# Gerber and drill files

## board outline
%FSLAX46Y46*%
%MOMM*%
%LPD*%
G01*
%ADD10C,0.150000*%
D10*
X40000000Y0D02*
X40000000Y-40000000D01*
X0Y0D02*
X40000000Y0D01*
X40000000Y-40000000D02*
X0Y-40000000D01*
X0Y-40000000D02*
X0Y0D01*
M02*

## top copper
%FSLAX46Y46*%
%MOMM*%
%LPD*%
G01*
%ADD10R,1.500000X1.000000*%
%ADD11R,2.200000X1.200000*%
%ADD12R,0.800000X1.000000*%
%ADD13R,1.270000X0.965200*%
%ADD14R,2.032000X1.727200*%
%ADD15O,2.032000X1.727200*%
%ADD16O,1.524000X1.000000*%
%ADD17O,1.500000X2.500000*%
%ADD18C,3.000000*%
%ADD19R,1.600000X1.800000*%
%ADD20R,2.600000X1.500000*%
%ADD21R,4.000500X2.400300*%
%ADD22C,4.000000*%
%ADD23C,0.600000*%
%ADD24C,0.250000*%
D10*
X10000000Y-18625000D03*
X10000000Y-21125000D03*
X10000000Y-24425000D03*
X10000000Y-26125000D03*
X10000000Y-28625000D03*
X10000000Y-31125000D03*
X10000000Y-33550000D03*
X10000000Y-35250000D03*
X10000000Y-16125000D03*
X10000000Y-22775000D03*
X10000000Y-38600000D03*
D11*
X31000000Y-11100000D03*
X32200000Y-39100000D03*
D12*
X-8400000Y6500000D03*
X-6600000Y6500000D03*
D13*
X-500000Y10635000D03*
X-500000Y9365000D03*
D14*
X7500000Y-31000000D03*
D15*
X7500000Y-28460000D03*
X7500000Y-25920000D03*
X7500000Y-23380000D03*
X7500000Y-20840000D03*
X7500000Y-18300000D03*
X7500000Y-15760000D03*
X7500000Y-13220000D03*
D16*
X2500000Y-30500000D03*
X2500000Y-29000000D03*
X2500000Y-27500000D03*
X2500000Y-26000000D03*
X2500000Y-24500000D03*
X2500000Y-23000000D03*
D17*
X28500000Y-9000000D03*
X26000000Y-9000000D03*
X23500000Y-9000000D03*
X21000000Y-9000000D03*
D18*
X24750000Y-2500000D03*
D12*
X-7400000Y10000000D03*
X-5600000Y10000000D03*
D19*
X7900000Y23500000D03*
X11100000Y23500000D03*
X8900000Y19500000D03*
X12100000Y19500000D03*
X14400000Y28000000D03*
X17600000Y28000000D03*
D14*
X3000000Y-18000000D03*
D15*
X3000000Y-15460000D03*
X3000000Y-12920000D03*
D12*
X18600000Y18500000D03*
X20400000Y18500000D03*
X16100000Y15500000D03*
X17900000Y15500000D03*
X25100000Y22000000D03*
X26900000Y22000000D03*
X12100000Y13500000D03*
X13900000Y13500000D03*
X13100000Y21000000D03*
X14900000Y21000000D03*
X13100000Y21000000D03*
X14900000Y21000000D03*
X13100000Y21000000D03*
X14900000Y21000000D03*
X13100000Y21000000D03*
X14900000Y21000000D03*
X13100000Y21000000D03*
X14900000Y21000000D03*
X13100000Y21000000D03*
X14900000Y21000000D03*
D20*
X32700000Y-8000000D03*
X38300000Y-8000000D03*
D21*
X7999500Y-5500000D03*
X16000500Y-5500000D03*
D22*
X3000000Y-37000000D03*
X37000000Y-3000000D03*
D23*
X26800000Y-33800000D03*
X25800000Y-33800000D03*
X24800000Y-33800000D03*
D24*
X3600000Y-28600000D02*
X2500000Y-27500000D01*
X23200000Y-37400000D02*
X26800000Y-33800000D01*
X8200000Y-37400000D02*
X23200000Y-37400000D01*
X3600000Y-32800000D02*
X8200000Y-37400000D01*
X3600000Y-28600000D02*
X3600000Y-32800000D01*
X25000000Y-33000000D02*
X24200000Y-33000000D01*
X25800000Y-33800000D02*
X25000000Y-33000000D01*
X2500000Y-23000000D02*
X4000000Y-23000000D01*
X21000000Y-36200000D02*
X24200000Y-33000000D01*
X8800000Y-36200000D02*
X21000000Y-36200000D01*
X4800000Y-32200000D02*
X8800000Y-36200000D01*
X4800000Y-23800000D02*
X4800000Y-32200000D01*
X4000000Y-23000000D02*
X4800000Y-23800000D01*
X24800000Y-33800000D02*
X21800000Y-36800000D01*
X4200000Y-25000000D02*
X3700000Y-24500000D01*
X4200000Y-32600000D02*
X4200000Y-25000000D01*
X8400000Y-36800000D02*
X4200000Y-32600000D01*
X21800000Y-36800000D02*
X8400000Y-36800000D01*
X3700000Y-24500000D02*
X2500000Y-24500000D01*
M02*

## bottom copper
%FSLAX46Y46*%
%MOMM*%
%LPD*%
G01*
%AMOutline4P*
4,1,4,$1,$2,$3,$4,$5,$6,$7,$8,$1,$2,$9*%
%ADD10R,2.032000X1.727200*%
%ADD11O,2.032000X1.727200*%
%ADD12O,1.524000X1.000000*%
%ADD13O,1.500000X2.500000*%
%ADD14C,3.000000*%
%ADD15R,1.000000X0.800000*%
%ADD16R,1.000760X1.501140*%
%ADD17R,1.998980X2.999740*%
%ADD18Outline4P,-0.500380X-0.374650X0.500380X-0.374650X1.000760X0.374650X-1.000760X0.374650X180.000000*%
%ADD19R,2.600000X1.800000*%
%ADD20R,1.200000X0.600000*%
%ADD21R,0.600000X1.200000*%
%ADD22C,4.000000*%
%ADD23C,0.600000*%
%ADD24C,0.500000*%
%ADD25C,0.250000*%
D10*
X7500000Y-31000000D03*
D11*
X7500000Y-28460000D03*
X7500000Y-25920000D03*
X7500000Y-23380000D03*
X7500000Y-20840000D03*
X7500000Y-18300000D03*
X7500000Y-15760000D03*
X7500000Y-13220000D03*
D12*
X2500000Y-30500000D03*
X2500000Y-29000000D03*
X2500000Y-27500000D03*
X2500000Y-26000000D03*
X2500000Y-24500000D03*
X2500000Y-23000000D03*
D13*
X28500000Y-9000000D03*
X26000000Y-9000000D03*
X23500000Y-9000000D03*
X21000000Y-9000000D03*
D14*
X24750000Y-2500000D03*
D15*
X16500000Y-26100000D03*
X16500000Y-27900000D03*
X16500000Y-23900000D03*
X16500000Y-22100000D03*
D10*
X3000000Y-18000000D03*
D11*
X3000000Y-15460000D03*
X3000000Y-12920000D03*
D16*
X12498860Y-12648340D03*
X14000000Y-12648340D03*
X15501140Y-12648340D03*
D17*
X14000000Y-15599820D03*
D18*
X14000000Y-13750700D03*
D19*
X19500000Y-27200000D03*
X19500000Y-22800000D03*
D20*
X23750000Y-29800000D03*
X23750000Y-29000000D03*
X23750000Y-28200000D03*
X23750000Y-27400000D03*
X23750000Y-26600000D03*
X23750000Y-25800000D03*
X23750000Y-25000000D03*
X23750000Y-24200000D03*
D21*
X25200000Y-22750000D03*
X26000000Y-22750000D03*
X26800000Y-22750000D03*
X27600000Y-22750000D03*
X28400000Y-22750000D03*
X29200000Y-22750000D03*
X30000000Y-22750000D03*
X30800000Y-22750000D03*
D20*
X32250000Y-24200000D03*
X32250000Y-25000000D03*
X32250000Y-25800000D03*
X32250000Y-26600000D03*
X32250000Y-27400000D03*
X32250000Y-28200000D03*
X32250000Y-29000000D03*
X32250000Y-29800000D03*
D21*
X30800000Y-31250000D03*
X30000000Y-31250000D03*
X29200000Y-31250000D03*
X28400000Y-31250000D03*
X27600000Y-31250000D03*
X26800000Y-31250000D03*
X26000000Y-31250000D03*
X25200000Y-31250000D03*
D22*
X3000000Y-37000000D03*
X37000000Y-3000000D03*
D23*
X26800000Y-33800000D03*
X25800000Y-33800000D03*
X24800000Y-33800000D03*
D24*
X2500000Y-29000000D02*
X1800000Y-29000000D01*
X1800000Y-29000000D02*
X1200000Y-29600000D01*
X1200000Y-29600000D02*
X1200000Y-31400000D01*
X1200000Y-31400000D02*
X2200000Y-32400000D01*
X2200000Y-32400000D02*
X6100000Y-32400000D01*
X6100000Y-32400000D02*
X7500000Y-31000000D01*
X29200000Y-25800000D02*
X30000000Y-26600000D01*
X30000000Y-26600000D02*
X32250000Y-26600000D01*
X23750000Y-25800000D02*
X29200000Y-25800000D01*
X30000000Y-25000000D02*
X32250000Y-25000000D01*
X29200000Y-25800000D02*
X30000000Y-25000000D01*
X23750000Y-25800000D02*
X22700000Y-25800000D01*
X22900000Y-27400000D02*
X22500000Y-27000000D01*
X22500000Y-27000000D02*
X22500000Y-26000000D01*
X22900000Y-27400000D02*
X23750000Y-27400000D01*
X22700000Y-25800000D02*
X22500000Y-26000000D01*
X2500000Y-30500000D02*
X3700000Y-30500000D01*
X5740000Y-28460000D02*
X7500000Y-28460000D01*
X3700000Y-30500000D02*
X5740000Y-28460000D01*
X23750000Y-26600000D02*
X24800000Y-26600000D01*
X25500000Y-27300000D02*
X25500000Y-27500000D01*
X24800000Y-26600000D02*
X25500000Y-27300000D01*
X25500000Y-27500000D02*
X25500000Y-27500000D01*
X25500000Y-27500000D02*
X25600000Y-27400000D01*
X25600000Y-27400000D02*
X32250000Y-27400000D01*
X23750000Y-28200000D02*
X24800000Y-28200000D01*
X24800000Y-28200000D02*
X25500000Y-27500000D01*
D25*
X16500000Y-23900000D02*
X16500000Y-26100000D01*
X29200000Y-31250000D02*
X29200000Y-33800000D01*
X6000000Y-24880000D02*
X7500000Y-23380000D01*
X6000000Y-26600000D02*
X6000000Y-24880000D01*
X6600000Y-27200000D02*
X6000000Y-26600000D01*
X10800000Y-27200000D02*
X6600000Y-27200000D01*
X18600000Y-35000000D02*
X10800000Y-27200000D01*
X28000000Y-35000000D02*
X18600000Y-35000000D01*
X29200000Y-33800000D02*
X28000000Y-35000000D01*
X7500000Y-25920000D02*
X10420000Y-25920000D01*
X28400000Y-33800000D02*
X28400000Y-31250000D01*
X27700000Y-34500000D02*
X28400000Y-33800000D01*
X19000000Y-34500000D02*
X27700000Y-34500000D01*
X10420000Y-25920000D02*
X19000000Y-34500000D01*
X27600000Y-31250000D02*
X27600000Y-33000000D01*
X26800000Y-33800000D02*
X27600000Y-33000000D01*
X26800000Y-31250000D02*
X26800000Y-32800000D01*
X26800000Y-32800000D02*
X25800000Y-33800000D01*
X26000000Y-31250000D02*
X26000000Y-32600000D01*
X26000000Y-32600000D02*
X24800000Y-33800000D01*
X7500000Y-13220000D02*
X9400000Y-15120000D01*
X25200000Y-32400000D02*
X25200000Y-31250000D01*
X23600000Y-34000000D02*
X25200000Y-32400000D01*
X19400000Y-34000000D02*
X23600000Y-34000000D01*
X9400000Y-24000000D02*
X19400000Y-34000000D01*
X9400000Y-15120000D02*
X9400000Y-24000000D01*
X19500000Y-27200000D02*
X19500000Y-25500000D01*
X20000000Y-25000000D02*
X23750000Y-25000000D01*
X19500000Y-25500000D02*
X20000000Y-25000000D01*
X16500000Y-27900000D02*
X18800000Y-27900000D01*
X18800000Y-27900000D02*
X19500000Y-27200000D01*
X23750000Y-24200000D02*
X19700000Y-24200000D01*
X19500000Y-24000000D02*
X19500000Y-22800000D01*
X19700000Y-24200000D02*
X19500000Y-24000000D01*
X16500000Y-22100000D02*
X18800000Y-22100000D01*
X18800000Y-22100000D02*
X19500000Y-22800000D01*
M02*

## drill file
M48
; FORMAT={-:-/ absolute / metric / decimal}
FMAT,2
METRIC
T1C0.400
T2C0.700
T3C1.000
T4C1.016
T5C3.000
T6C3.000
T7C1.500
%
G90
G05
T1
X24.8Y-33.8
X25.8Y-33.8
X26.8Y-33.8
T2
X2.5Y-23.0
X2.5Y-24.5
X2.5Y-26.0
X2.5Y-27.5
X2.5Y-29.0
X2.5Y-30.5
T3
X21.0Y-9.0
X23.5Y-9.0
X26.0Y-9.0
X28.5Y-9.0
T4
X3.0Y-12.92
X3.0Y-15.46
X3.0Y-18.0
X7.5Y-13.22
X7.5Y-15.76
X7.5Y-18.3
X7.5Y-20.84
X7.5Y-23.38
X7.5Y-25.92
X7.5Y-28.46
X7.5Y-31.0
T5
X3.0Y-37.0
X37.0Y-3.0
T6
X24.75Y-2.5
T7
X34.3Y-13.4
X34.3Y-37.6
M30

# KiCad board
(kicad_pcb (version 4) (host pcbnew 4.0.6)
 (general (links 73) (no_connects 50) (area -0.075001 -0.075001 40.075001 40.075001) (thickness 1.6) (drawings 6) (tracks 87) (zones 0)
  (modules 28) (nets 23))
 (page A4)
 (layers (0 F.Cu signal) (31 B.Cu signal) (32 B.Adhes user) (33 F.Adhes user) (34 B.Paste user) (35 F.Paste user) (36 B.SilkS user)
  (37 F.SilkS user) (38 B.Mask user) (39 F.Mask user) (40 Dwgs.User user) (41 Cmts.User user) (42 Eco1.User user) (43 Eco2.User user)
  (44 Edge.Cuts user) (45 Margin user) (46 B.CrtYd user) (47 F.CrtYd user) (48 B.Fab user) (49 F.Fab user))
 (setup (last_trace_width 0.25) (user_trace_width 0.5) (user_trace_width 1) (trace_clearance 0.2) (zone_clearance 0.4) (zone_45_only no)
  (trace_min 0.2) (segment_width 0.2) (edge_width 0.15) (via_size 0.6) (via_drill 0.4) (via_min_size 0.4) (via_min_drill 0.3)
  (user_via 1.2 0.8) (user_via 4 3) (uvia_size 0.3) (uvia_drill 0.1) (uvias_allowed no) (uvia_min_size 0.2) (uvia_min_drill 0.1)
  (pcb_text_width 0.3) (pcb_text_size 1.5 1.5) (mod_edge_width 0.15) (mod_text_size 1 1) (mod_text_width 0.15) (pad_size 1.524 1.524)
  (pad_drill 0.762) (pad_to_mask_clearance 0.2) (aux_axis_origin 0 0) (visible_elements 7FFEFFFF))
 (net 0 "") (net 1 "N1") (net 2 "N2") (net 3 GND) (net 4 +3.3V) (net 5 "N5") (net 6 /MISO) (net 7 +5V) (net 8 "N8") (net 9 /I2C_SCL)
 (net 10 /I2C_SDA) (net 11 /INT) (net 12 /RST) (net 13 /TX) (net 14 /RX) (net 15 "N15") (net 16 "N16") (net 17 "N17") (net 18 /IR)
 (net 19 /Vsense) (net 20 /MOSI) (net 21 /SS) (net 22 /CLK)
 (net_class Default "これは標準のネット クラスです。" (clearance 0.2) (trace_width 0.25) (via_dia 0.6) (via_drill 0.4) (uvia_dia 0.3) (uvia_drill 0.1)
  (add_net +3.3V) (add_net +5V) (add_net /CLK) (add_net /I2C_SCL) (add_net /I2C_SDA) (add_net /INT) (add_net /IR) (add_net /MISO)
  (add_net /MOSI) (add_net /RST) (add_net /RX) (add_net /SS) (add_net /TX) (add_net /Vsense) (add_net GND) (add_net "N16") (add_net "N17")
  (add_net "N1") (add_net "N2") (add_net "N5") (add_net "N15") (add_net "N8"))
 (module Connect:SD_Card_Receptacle (layer F.Cu) (at 10 25.5 90)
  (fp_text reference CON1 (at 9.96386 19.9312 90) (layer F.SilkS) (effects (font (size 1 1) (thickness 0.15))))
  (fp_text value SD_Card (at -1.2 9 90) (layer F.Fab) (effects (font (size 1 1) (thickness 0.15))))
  (pad 1 smd rect (at 6.875 0 90) (size 1 1.5) (layers F.Cu F.Paste F.Mask) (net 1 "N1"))
  (pad 2 smd rect (at 4.375 0 90) (size 1 1.5) (layers F.Cu F.Paste F.Mask) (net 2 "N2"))
  (pad 3 smd rect (at 1.075 0 90) (size 1 1.5) (layers F.Cu F.Paste F.Mask) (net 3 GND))
  (pad 4 smd rect (at -0.625 0 90) (size 1 1.5) (layers F.Cu F.Paste F.Mask) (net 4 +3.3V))
  (pad 5 smd rect (at -3.125 0 90) (size 1 1.5) (layers F.Cu F.Paste F.Mask) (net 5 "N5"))
  (pad 6 smd rect (at -5.625 0 90) (size 1 1.5) (layers F.Cu F.Paste F.Mask) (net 3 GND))
  (pad 7 smd rect (at -8.05 0 90) (size 1 1.5) (layers F.Cu F.Paste F.Mask) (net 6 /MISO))
  (pad 8 smd rect (at -9.75 0 90) (size 1 1.5) (layers F.Cu F.Paste F.Mask))
  (pad 9 smd rect (at 9.375 0 90) (size 1 1.5) (layers F.Cu F.Paste F.Mask))
  (pad 10 smd rect (at 2.725 0 90) (size 1 1.5) (layers F.Cu F.Paste F.Mask))
  (pad 11 smd rect (at -13.1 0 90) (size 1 1.5) (layers F.Cu F.Paste F.Mask))
  (pad 12 smd rect (at 14.4 21 90) (size 1.2 2.2) (layers F.Cu F.Paste F.Mask) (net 3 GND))
  (pad 13 smd rect (at -13.6 22.2 90) (size 1.2 2.2) (layers F.Cu F.Paste F.Mask) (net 3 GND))
  (pad "" np_thru_hole circle (at 12.1 24.3 90) (size 1.5 1.5) (drill 1.5) (layers *.Cu *.Mask F.SilkS))
  (pad "" np_thru_hole circle (at -12.1 24.3 90) (size 1.5 1.5) (drill 1.5) (layers *.Cu *.Mask F.SilkS)))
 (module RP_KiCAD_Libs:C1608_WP (layer F.Cu) (at -7.5 -6.5)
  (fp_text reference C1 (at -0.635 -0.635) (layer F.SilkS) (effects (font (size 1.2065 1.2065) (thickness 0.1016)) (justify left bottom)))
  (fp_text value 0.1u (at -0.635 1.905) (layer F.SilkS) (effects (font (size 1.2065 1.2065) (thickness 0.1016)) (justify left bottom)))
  (pad 1 smd rect (at -0.9 0) (size 0.8 1) (layers F.Cu F.Paste F.Mask) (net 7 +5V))
  (pad 2 smd rect (at 0.9 0) (size 0.8 1) (layers F.Cu F.Paste F.Mask) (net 3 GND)))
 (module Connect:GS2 (layer F.Cu) (at -0.5 -10)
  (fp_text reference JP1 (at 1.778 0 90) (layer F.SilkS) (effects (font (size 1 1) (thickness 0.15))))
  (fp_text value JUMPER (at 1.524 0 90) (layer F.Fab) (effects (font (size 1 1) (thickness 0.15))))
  (pad 1 smd rect (at 0 -0.635) (size 1.27 0.9652) (layers F.Cu F.Paste F.Mask) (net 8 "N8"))
  (pad 2 smd rect (at 0 0.635) (size 1.27 0.9652) (layers F.Cu F.Paste F.Mask) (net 3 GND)))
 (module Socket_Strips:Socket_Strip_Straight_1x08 (layer F.Cu) (at 7.5 31 90)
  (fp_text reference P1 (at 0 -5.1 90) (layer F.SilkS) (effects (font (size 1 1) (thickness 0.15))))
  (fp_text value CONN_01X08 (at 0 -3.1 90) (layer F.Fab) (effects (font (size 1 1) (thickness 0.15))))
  (pad 1 thru_hole rect (at 0 0 90) (size 1.7272 2.032) (drill 1.016) (layers *.Cu *.Mask F.SilkS) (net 7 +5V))
  (pad 2 thru_hole oval (at 2.54 0 90) (size 1.7272 2.032) (drill 1.016) (layers *.Cu *.Mask F.SilkS) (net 3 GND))
  (pad 3 thru_hole oval (at 5.08 0 90) (size 1.7272 2.032) (drill 1.016) (layers *.Cu *.Mask F.SilkS) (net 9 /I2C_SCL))
  (pad 4 thru_hole oval (at 7.62 0 90) (size 1.7272 2.032) (drill 1.016) (layers *.Cu *.Mask F.SilkS) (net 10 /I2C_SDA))
  (pad 5 thru_hole oval (at 10.16 0 90) (size 1.7272 2.032) (drill 1.016) (layers *.Cu *.Mask F.SilkS))
  (pad 6 thru_hole oval (at 12.7 0 90) (size 1.7272 2.032) (drill 1.016) (layers *.Cu *.Mask F.SilkS))
  (pad 7 thru_hole oval (at 15.24 0 90) (size 1.7272 2.032) (drill 1.016) (layers *.Cu *.Mask F.SilkS) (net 8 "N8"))
  (pad 8 thru_hole oval (at 17.78 0 90) (size 1.7272 2.032) (drill 1.016) (layers *.Cu *.Mask F.SilkS) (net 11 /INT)))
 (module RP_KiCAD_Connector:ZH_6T (layer F.Cu) (at 2.5 30.5 90)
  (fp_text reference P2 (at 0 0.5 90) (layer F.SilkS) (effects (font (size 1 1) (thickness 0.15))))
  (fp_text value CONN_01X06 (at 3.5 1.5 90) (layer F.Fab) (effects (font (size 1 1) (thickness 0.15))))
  (pad 1 thru_hole oval (at 0 0 90) (size 1 1.524) (drill 0.7) (layers *.Cu *.Mask) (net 3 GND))
  (pad 2 thru_hole oval (at 1.5 0 90) (size 1 1.524) (drill 0.7) (layers *.Cu *.Mask) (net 7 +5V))
  (pad 3 thru_hole oval (at 3 0 90) (size 1 1.524) (drill 0.7) (layers *.Cu *.Mask) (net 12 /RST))
  (pad 4 thru_hole oval (at 4.5 0 90) (size 1 1.524) (drill 0.7) (layers *.Cu *.Mask))
  (pad 5 thru_hole oval (at 6 0 90) (size 1 1.524) (drill 0.7) (layers *.Cu *.Mask) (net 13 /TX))
  (pad 6 thru_hole oval (at 7.5 0 90) (size 1 1.524) (drill 0.7) (layers *.Cu *.Mask) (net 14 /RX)))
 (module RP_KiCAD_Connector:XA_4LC (layer F.Cu) (at 28.5 9 180)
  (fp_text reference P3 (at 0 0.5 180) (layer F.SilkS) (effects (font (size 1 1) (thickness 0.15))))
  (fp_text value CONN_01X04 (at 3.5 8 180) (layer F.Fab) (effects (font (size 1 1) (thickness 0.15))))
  (pad 1 thru_hole oval (at 0 0 180) (size 1.5 2.5) (drill 1) (layers *.Cu *.Mask F.SilkS) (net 3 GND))
  (pad 2 thru_hole oval (at 2.5 0 180) (size 1.5 2.5) (drill 1) (layers *.Cu *.Mask F.SilkS) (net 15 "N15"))
  (pad 3 thru_hole oval (at 5 0 180) (size 1.5 2.5) (drill 1) (layers *.Cu *.Mask F.SilkS) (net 14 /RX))
  (pad 4 thru_hole oval (at 7.5 0 180) (size 1.5 2.5) (drill 1) (layers *.Cu *.Mask F.SilkS) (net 13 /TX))
  (pad "" thru_hole circle (at 3.75 6.5 180) (size 3 3) (drill 3) (layers *.Cu *.Mask F.SilkS) (clearance -0.3)))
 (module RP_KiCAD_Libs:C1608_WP (layer F.Cu) (at -6.5 -10)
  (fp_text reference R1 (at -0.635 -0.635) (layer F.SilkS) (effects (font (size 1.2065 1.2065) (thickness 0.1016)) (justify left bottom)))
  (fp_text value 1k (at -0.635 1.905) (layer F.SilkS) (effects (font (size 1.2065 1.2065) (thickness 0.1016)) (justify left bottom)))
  (pad 1 smd rect (at -0.9 0) (size 0.8 1) (layers F.Cu F.Paste F.Mask) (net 7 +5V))
  (pad 2 smd rect (at 0.9 0) (size 0.8 1) (layers F.Cu F.Paste F.Mask) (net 12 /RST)))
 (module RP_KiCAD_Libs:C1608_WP (layer B.Cu) (at 16.5 27 270)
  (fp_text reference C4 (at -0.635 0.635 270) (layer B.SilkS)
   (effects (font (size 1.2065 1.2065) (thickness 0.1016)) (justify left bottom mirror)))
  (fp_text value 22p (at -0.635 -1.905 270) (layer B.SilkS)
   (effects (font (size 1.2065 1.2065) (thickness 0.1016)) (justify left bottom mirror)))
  (pad 1 smd rect (at -0.9 0 270) (size 0.8 1) (layers B.Cu B.Paste B.Mask) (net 3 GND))
  (pad 2 smd rect (at 0.9 0 270) (size 0.8 1) (layers B.Cu B.Paste B.Mask) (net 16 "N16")))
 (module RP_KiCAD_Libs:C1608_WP (layer B.Cu) (at 16.5 23 90)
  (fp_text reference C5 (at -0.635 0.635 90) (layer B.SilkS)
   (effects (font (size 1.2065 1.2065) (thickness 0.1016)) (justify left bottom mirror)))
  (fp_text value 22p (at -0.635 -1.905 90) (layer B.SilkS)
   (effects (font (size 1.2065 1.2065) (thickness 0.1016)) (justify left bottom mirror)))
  (pad 1 smd rect (at -0.9 0 90) (size 0.8 1) (layers B.Cu B.Paste B.Mask) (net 3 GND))
  (pad 2 smd rect (at 0.9 0 90) (size 0.8 1) (layers B.Cu B.Paste B.Mask) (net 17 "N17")))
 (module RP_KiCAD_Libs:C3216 (layer F.Cu) (at 9.5 -23.5)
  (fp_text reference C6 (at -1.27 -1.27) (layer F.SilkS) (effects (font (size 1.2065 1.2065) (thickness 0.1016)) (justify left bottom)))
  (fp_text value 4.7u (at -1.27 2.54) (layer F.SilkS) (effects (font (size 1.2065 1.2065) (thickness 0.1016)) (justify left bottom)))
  (pad 1 smd rect (at -1.6 0) (size 1.6 1.8) (layers F.Cu F.Paste F.Mask) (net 7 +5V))
  (pad 2 smd rect (at 1.6 0) (size 1.6 1.8) (layers F.Cu F.Paste F.Mask) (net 3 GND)))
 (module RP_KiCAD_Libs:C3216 (layer F.Cu) (at 10.5 -19.5)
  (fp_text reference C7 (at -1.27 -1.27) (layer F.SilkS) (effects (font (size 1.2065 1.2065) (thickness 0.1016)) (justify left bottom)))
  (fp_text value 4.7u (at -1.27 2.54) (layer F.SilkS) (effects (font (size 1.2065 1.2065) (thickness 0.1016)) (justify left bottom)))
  (pad 1 smd rect (at -1.6 0) (size 1.6 1.8) (layers F.Cu F.Paste F.Mask) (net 4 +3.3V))
  (pad 2 smd rect (at 1.6 0) (size 1.6 1.8) (layers F.Cu F.Paste F.Mask) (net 3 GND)))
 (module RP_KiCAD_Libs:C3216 (layer F.Cu) (at 16 -28)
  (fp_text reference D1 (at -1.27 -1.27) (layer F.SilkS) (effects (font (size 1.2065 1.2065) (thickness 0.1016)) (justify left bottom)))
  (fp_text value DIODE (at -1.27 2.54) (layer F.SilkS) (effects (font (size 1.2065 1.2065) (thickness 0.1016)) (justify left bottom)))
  (pad 1 smd rect (at -1.6 0) (size 1.6 1.8) (layers F.Cu F.Paste F.Mask) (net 7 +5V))
  (pad 2 smd rect (at 1.6 0) (size 1.6 1.8) (layers F.Cu F.Paste F.Mask) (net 15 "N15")))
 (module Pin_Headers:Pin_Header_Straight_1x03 (layer F.Cu) (at 3 18 180)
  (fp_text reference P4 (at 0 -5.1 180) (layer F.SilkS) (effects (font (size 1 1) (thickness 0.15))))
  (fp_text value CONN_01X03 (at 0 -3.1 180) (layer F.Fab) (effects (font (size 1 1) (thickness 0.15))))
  (pad 1 thru_hole rect (at 0 0 180) (size 2.032 1.7272) (drill 1.016) (layers *.Cu *.Mask F.SilkS) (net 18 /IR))
  (pad 2 thru_hole oval (at 0 2.54 180) (size 2.032 1.7272) (drill 1.016) (layers *.Cu *.Mask F.SilkS) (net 3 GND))
  (pad 3 thru_hole oval (at 0 5.08 180) (size 2.032 1.7272) (drill 1.016) (layers *.Cu *.Mask F.SilkS) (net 7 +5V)))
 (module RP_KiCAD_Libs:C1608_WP (layer F.Cu) (at 19.5 -18.5)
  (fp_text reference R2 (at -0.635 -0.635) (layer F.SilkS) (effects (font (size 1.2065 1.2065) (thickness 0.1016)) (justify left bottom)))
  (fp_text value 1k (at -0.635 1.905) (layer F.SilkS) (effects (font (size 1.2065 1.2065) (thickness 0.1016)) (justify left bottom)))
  (pad 1 smd rect (at -0.9 0) (size 0.8 1) (layers F.Cu F.Paste F.Mask) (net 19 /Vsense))
  (pad 2 smd rect (at 0.9 0) (size 0.8 1) (layers F.Cu F.Paste F.Mask) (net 15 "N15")))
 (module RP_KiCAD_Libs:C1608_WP (layer F.Cu) (at 17 -15.5)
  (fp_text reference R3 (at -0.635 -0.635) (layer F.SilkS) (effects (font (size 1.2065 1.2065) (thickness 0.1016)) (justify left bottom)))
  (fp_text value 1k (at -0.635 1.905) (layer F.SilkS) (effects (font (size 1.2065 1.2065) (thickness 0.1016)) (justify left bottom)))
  (pad 1 smd rect (at -0.9 0) (size 0.8 1) (layers F.Cu F.Paste F.Mask) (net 10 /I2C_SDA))
  (pad 2 smd rect (at 0.9 0) (size 0.8 1) (layers F.Cu F.Paste F.Mask) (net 7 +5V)))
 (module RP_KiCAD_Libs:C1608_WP (layer F.Cu) (at 26 -22)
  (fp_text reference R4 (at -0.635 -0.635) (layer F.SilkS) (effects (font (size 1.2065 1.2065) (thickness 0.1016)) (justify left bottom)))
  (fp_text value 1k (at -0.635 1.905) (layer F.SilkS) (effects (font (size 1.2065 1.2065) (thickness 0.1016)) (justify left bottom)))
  (pad 1 smd rect (at -0.9 0) (size 0.8 1) (layers F.Cu F.Paste F.Mask) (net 9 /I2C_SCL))
  (pad 2 smd rect (at 0.9 0) (size 0.8 1) (layers F.Cu F.Paste F.Mask) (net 7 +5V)))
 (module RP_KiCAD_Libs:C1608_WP (layer F.Cu) (at 13 -13.5)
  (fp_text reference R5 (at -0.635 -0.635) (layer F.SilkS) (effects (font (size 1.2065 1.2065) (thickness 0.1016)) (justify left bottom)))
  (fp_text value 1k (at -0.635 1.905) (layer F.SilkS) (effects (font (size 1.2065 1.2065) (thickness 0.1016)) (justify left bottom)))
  (pad 1 smd rect (at -0.9 0) (size 0.8 1) (layers F.Cu F.Paste F.Mask) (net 3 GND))
  (pad 2 smd rect (at 0.9 0) (size 0.8 1) (layers F.Cu F.Paste F.Mask) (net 19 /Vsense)))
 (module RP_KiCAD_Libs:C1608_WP (layer F.Cu) (at 14 -21)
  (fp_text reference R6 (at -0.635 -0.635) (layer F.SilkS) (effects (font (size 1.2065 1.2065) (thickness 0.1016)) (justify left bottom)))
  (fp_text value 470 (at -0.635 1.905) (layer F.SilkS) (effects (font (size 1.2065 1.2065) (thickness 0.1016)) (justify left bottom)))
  (pad 1 smd rect (at -0.9 0) (size 0.8 1) (layers F.Cu F.Paste F.Mask) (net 2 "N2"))
  (pad 2 smd rect (at 0.9 0) (size 0.8 1) (layers F.Cu F.Paste F.Mask) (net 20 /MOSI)))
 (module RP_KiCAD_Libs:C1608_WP (layer F.Cu) (at 14 -21)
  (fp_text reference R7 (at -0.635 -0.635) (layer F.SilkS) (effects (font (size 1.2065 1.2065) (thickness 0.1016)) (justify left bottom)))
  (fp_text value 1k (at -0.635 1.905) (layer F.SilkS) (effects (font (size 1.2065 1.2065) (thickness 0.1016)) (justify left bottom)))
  (pad 1 smd rect (at -0.9 0) (size 0.8 1) (layers F.Cu F.Paste F.Mask) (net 2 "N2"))
  (pad 2 smd rect (at 0.9 0) (size 0.8 1) (layers F.Cu F.Paste F.Mask) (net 3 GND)))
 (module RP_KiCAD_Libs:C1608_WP (layer F.Cu) (at 14 -21)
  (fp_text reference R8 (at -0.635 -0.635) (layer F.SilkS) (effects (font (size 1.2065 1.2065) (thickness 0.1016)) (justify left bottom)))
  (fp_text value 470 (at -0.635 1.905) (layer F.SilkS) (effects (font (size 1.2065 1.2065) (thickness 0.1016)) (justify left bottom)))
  (pad 1 smd rect (at -0.9 0) (size 0.8 1) (layers F.Cu F.Paste F.Mask) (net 1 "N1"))
  (pad 2 smd rect (at 0.9 0) (size 0.8 1) (layers F.Cu F.Paste F.Mask) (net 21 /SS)))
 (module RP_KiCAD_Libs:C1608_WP (layer F.Cu) (at 14 -21)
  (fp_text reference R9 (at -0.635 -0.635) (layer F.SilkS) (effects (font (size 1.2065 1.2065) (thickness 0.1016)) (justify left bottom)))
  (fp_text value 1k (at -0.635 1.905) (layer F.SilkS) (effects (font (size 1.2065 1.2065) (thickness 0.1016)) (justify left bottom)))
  (pad 1 smd rect (at -0.9 0) (size 0.8 1) (layers F.Cu F.Paste F.Mask) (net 1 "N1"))
  (pad 2 smd rect (at 0.9 0) (size 0.8 1) (layers F.Cu F.Paste F.Mask) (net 3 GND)))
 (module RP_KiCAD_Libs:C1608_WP (layer F.Cu) (at 14 -21)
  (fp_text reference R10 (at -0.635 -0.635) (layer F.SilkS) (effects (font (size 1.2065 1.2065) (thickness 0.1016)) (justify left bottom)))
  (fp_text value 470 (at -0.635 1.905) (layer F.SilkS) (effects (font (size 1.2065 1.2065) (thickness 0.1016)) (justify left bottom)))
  (pad 1 smd rect (at -0.9 0) (size 0.8 1) (layers F.Cu F.Paste F.Mask) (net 5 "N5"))
  (pad 2 smd rect (at 0.9 0) (size 0.8 1) (layers F.Cu F.Paste F.Mask) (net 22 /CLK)))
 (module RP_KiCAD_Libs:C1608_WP (layer F.Cu) (at 14 -21)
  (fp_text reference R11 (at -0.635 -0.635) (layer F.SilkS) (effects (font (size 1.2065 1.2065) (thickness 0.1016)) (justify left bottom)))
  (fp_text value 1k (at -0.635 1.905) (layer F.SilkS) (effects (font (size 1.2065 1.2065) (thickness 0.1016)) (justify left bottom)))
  (pad 1 smd rect (at -0.9 0) (size 0.8 1) (layers F.Cu F.Paste F.Mask) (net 5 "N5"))
  (pad 2 smd rect (at 0.9 0) (size 0.8 1) (layers F.Cu F.Paste F.Mask) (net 3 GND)))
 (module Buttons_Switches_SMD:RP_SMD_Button (layer F.Cu) (at 35.5 8 180)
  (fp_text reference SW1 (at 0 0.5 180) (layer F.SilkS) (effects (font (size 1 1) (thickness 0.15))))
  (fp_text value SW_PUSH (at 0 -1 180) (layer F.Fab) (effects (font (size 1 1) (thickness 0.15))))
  (pad 1 smd rect (at 2.8 0 180) (size 2.6 1.5) (layers F.Cu F.Paste F.Mask) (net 12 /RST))
  (pad 2 smd rect (at -2.8 0 180) (size 2.6 1.5) (layers F.Cu F.Paste F.Mask) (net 3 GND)))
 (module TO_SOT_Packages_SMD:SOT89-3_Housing (layer B.Cu) (at 14 14.5)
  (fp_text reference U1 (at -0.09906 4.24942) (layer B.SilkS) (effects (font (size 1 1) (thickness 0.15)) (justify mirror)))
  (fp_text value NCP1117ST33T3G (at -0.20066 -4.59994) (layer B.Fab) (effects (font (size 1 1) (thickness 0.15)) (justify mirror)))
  (pad 1 smd rect (at -1.50114 -1.85166) (size 1.00076 1.50114) (layers B.Cu B.Paste B.Mask) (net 3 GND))
  (pad 2 smd rect (at 0 -1.85166) (size 1.00076 1.50114) (layers B.Cu B.Paste B.Mask) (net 4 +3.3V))
  (pad 3 smd rect (at 1.50114 -1.85166) (size 1.00076 1.50114) (layers B.Cu B.Paste B.Mask) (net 7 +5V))
  (pad 2 smd rect (at 0 1.09982) (size 1.99898 2.99974) (layers B.Cu B.Paste B.Mask) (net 4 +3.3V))
  (pad 2 smd trapezoid (at 0 -0.7493 180) (size 1.50114 0.7493) (rect_delta 0 -0.50038) (layers B.Cu B.Paste B.Mask) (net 4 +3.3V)))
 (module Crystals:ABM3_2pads (layer B.Cu) (at 19.5 25 90)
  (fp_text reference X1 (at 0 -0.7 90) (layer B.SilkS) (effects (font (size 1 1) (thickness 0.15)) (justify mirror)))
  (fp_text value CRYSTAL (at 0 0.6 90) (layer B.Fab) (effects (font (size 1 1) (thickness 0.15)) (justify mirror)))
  (pad 1 smd rect (at -2.2 0 90) (size 1.8 2.6) (layers B.Cu B.Paste B.Mask) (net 16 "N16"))
  (pad 2 smd rect (at 2.2 0 90) (size 1.8 2.6) (layers B.Cu B.Paste B.Mask) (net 17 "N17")))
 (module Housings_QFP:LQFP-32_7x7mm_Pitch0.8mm (layer B.Cu) (at 28 27)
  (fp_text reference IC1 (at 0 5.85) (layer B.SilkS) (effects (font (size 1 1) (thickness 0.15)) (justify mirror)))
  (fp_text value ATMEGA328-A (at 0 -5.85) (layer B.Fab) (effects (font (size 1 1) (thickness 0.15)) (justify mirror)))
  (pad 1 smd rect (at -4.25 2.8) (size 1.2 0.6) (layers B.Cu B.Paste B.Mask) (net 18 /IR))
  (pad 2 smd rect (at -4.25 2) (size 1.2 0.6) (layers B.Cu B.Paste B.Mask))
  (pad 3 smd rect (at -4.25 1.2) (size 1.2 0.6) (layers B.Cu B.Paste B.Mask) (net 3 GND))
  (pad 4 smd rect (at -4.25 0.4) (size 1.2 0.6) (layers B.Cu B.Paste B.Mask) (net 7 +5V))
  (pad 5 smd rect (at -4.25 -0.4) (size 1.2 0.6) (layers B.Cu B.Paste B.Mask) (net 3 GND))
  (pad 6 smd rect (at -4.25 -1.2) (size 1.2 0.6) (layers B.Cu B.Paste B.Mask) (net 7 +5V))
  (pad 7 smd rect (at -4.25 -2) (size 1.2 0.6) (layers B.Cu B.Paste B.Mask) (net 16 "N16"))
  (pad 8 smd rect (at -4.25 -2.8) (size 1.2 0.6) (layers B.Cu B.Paste B.Mask) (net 17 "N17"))
  (pad 9 smd rect (at -2.8 -4.25 270) (size 1.2 0.6) (layers B.Cu B.Paste B.Mask))
  (pad 10 smd rect (at -2 -4.25 270) (size 1.2 0.6) (layers B.Cu B.Paste B.Mask))
  (pad 11 smd rect (at -1.2 -4.25 270) (size 1.2 0.6) (layers B.Cu B.Paste B.Mask))
  (pad 12 smd rect (at -0.4 -4.25 270) (size 1.2 0.6) (layers B.Cu B.Paste B.Mask))
  (pad 13 smd rect (at 0.4 -4.25 270) (size 1.2 0.6) (layers B.Cu B.Paste B.Mask))
  (pad 14 smd rect (at 1.2 -4.25 270) (size 1.2 0.6) (layers B.Cu B.Paste B.Mask) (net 21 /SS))
  (pad 15 smd rect (at 2 -4.25 270) (size 1.2 0.6) (layers B.Cu B.Paste B.Mask) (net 20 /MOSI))
  (pad 16 smd rect (at 2.8 -4.25 270) (size 1.2 0.6) (layers B.Cu B.Paste B.Mask) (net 6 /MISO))
  (pad 17 smd rect (at 4.25 -2.8) (size 1.2 0.6) (layers B.Cu B.Paste B.Mask) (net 22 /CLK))
  (pad 18 smd rect (at 4.25 -2) (size 1.2 0.6) (layers B.Cu B.Paste B.Mask) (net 7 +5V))
  (pad 19 smd rect (at 4.25 -1.2) (size 1.2 0.6) (layers B.Cu B.Paste B.Mask))
  (pad 20 smd rect (at 4.25 -0.4) (size 1.2 0.6) (layers B.Cu B.Paste B.Mask) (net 7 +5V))
  (pad 21 smd rect (at 4.25 0.4) (size 1.2 0.6) (layers B.Cu B.Paste B.Mask) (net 3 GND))
  (pad 22 smd rect (at 4.25 1.2) (size 1.2 0.6) (layers B.Cu B.Paste B.Mask))
  (pad 23 smd rect (at 4.25 2) (size 1.2 0.6) (layers B.Cu B.Paste B.Mask))
  (pad 24 smd rect (at 4.25 2.8) (size 1.2 0.6) (layers B.Cu B.Paste B.Mask))
  (pad 25 smd rect (at 2.8 4.25 270) (size 1.2 0.6) (layers B.Cu B.Paste B.Mask))
  (pad 26 smd rect (at 2 4.25 270) (size 1.2 0.6) (layers B.Cu B.Paste B.Mask) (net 19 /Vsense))
  (pad 27 smd rect (at 1.2 4.25 270) (size 1.2 0.6) (layers B.Cu B.Paste B.Mask) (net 10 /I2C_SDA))
  (pad 28 smd rect (at 0.4 4.25 270) (size 1.2 0.6) (layers B.Cu B.Paste B.Mask) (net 9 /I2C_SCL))
  (pad 29 smd rect (at -0.4 4.25 270) (size 1.2 0.6) (layers B.Cu B.Paste B.Mask) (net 12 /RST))
  (pad 30 smd rect (at -1.2 4.25 270) (size 1.2 0.6) (layers B.Cu B.Paste B.Mask) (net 14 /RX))
  (pad 31 smd rect (at -2 4.25 270) (size 1.2 0.6) (layers B.Cu B.Paste B.Mask) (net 13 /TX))
  (pad 32 smd rect (at -2.8 4.25 270) (size 1.2 0.6) (layers B.Cu B.Paste B.Mask) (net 11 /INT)))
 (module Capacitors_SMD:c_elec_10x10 (layer F.Cu) (at 12 5.5 180)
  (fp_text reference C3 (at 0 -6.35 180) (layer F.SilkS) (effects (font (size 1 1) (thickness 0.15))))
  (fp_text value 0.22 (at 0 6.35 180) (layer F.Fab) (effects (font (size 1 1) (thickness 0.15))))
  (pad 1 smd rect (at 4.0005 0 180) (size 4.0005 2.4003) (layers F.Cu F.Paste F.Mask) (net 7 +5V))
  (pad 2 smd rect (at -4.0005 0 180) (size 4.0005 2.4003) (layers F.Cu F.Paste F.Mask) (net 3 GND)))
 (gr_line (start 40 0) (end 40 40) (angle 90) (layer Edge.Cuts) (width 0.15))
 (gr_line (start 0 0) (end 40 0) (angle 90) (layer Edge.Cuts) (width 0.15))
 (gr_line (start 40 40) (end 0 40) (angle 90) (layer Edge.Cuts) (width 0.15))
 (gr_line (start 0 40) (end 0 0) (angle 90) (layer Edge.Cuts) (width 0.15))
 (via (at 3 37) (size 4) (drill 3) (layers F.Cu B.Cu) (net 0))
 (via (at 37 3) (size 4) (drill 3) (layers F.Cu B.Cu) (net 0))
 (segment (start 2.5 29) (end 1.8 29) (width 0.5) (layer B.Cu) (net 7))
 (segment (start 1.8 29) (end 1.2 29.6) (width 0.5) (layer B.Cu) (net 7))
 (segment (start 1.2 29.6) (end 1.2 31.4) (width 0.5) (layer B.Cu) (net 7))
 (segment (start 1.2 31.4) (end 2.2 32.4) (width 0.5) (layer B.Cu) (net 7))
 (segment (start 2.2 32.4) (end 6.1 32.4) (width 0.5) (layer B.Cu) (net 7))
 (segment (start 6.1 32.4) (end 7.5 31) (width 0.5) (layer B.Cu) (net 7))
 (segment (start 29.2 25.8) (end 30 26.6) (width 0.5) (layer B.Cu) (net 7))
 (segment (start 30 26.6) (end 32.25 26.6) (width 0.5) (layer B.Cu) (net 7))
 (segment (start 23.75 25.8) (end 29.2 25.8) (width 0.5) (layer B.Cu) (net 7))
 (segment (start 30 25) (end 32.25 25) (width 0.5) (layer B.Cu) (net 7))
 (segment (start 29.2 25.8) (end 30 25) (width 0.5) (layer B.Cu) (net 7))
 (segment (start 23.75 25.8) (end 22.7 25.8) (width 0.5) (layer B.Cu) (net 7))
 (segment (start 22.9 27.4) (end 22.5 27) (width 0.5) (layer B.Cu) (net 7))
 (segment (start 22.5 27) (end 22.5 26) (width 0.5) (layer B.Cu) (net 7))
 (segment (start 22.9 27.4) (end 23.75 27.4) (width 0.5) (layer B.Cu) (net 7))
 (segment (start 22.7 25.8) (end 22.5 26) (width 0.5) (layer B.Cu) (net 7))
 (segment (start 2.5 30.5) (end 3.7 30.5) (width 0.5) (layer B.Cu) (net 3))
 (segment (start 5.74 28.46) (end 7.5 28.46) (width 0.5) (layer B.Cu) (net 3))
 (segment (start 3.7 30.5) (end 5.74 28.46) (width 0.5) (layer B.Cu) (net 3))
 (segment (start 23.75 26.6) (end 24.8 26.6) (width 0.5) (layer B.Cu) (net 3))
 (segment (start 25.5 27.3) (end 25.5 27.5) (width 0.5) (layer B.Cu) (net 3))
 (segment (start 24.8 26.6) (end 25.5 27.3) (width 0.5) (layer B.Cu) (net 3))
 (segment (start 25.5 27.5) (end 25.5 27.5) (width 0.5) (layer B.Cu) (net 3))
 (segment (start 25.5 27.5) (end 25.6 27.4) (width 0.5) (layer B.Cu) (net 3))
 (segment (start 25.6 27.4) (end 32.25 27.4) (width 0.5) (layer B.Cu) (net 3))
 (segment (start 23.75 28.2) (end 24.8 28.2) (width 0.5) (layer B.Cu) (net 3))
 (segment (start 24.8 28.2) (end 25.5 27.5) (width 0.5) (layer B.Cu) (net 3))
 (segment (start 16.5 23.9) (end 16.5 26.1) (width 0.25) (layer B.Cu) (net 3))
 (segment (start 29.2 31.25) (end 29.2 33.8) (width 0.25) (layer B.Cu) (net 10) (status 400000))
 (segment (start 6 24.88) (end 7.5 23.38) (width 0.25) (layer B.Cu) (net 10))
 (segment (start 6 26.6) (end 6 24.88) (width 0.25) (layer B.Cu) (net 10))
 (segment (start 6.6 27.2) (end 6 26.6) (width 0.25) (layer B.Cu) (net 10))
 (segment (start 10.8 27.2) (end 6.6 27.2) (width 0.25) (layer B.Cu) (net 10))
 (segment (start 18.6 35) (end 10.8 27.2) (width 0.25) (layer B.Cu) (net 10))
 (segment (start 28 35) (end 18.6 35) (width 0.25) (layer B.Cu) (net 10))
 (segment (start 29.2 33.8) (end 28 35) (width 0.25) (layer B.Cu) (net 10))
 (segment (start 7.5 25.92) (end 10.42 25.92) (width 0.25) (layer B.Cu) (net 9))
 (segment (start 28.4 33.8) (end 28.4 31.25) (width 0.25) (layer B.Cu) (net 9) (status 800000))
 (segment (start 27.7 34.5) (end 28.4 33.8) (width 0.25) (layer B.Cu) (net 9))
 (segment (start 19 34.5) (end 27.7 34.5) (width 0.25) (layer B.Cu) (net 9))
 (segment (start 10.42 25.92) (end 19 34.5) (width 0.25) (layer B.Cu) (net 9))
 (segment (start 27.6 31.25) (end 27.6 33) (width 0.25) (layer B.Cu) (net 12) (status 400000))
 (segment (start 26.8 33.8) (end 27.6 33) (width 0.25) (layer B.Cu) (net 12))
 (segment (start 3.6 28.6) (end 2.5 27.5) (width 0.25) (layer F.Cu) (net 12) (status 800000))
 (segment (start 23.2 37.4) (end 26.8 33.8) (width 0.25) (layer F.Cu) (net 12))
 (segment (start 8.2 37.4) (end 23.2 37.4) (width 0.25) (layer F.Cu) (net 12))
 (segment (start 3.6 32.8) (end 8.2 37.4) (width 0.25) (layer F.Cu) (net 12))
 (segment (start 3.6 28.6) (end 3.6 32.8) (width 0.25) (layer F.Cu) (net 12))
 (via (at 26.8 33.8) (size 0.6) (drill 0.4) (layers F.Cu B.Cu) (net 12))
 (segment (start 26.8 31.25) (end 26.8 32.8) (width 0.25) (layer B.Cu) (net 14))
 (segment (start 25 33) (end 24.2 33) (width 0.25) (layer F.Cu) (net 14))
 (segment (start 25.8 33.8) (end 25 33) (width 0.25) (layer F.Cu) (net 14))
 (via (at 25.8 33.8) (size 0.6) (drill 0.4) (layers F.Cu B.Cu) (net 14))
 (segment (start 26.8 32.8) (end 25.8 33.8) (width 0.25) (layer B.Cu) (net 14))
 (segment (start 2.5 23) (end 4 23) (width 0.25) (layer F.Cu) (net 14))
 (segment (start 21 36.2) (end 24.2 33) (width 0.25) (layer F.Cu) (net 14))
 (segment (start 8.8 36.2) (end 21 36.2) (width 0.25) (layer F.Cu) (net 14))
 (segment (start 4.8 32.2) (end 8.8 36.2) (width 0.25) (layer F.Cu) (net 14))
 (segment (start 4.8 23.8) (end 4.8 32.2) (width 0.25) (layer F.Cu) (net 14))
 (segment (start 4 23) (end 4.8 23.8) (width 0.25) (layer F.Cu) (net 14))
 (segment (start 26 31.25) (end 26 32.6) (width 0.25) (layer B.Cu) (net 13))
 (segment (start 24.8 33.8) (end 21.8 36.8) (width 0.25) (layer F.Cu) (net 13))
 (via (at 24.8 33.8) (size 0.6) (drill 0.4) (layers F.Cu B.Cu) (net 13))
 (segment (start 26 32.6) (end 24.8 33.8) (width 0.25) (layer B.Cu) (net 13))
 (segment (start 4.2 25) (end 3.7 24.5) (width 0.25) (layer F.Cu) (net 13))
 (segment (start 4.2 32.6) (end 4.2 25) (width 0.25) (layer F.Cu) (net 13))
 (segment (start 8.4 36.8) (end 4.2 32.6) (width 0.25) (layer F.Cu) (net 13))
 (segment (start 21.8 36.8) (end 8.4 36.8) (width 0.25) (layer F.Cu) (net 13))
 (segment (start 3.7 24.5) (end 2.5 24.5) (width 0.25) (layer F.Cu) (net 13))
 (segment (start 7.5 13.22) (end 9.4 15.12) (width 0.25) (layer B.Cu) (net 11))
 (segment (start 25.2 32.4) (end 25.2 31.25) (width 0.25) (layer B.Cu) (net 11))
 (segment (start 23.6 34) (end 25.2 32.4) (width 0.25) (layer B.Cu) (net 11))
 (segment (start 19.4 34) (end 23.6 34) (width 0.25) (layer B.Cu) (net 11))
 (segment (start 9.4 24) (end 19.4 34) (width 0.25) (layer B.Cu) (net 11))
 (segment (start 9.4 15.12) (end 9.4 24) (width 0.25) (layer B.Cu) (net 11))
 (segment (start 19.5 27.2) (end 19.5 25.5) (width 0.25) (layer B.Cu) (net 16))
 (segment (start 20 25) (end 23.75 25) (width 0.25) (layer B.Cu) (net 16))
 (segment (start 19.5 25.5) (end 20 25) (width 0.25) (layer B.Cu) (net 16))
 (segment (start 16.5 27.9) (end 18.8 27.9) (width 0.25) (layer B.Cu) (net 16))
 (segment (start 18.8 27.9) (end 19.5 27.2) (width 0.25) (layer B.Cu) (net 16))
 (segment (start 23.75 24.2) (end 19.7 24.2) (width 0.25) (layer B.Cu) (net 17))
 (segment (start 19.5 24) (end 19.5 22.8) (width 0.25) (layer B.Cu) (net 17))
 (segment (start 19.7 24.2) (end 19.5 24) (width 0.25) (layer B.Cu) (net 17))
 (segment (start 16.5 22.1) (end 18.8 22.1) (width 0.25) (layer B.Cu) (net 17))
 (segment (start 18.8 22.1) (end 19.5 22.8) (width 0.25) (layer B.Cu) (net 17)))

